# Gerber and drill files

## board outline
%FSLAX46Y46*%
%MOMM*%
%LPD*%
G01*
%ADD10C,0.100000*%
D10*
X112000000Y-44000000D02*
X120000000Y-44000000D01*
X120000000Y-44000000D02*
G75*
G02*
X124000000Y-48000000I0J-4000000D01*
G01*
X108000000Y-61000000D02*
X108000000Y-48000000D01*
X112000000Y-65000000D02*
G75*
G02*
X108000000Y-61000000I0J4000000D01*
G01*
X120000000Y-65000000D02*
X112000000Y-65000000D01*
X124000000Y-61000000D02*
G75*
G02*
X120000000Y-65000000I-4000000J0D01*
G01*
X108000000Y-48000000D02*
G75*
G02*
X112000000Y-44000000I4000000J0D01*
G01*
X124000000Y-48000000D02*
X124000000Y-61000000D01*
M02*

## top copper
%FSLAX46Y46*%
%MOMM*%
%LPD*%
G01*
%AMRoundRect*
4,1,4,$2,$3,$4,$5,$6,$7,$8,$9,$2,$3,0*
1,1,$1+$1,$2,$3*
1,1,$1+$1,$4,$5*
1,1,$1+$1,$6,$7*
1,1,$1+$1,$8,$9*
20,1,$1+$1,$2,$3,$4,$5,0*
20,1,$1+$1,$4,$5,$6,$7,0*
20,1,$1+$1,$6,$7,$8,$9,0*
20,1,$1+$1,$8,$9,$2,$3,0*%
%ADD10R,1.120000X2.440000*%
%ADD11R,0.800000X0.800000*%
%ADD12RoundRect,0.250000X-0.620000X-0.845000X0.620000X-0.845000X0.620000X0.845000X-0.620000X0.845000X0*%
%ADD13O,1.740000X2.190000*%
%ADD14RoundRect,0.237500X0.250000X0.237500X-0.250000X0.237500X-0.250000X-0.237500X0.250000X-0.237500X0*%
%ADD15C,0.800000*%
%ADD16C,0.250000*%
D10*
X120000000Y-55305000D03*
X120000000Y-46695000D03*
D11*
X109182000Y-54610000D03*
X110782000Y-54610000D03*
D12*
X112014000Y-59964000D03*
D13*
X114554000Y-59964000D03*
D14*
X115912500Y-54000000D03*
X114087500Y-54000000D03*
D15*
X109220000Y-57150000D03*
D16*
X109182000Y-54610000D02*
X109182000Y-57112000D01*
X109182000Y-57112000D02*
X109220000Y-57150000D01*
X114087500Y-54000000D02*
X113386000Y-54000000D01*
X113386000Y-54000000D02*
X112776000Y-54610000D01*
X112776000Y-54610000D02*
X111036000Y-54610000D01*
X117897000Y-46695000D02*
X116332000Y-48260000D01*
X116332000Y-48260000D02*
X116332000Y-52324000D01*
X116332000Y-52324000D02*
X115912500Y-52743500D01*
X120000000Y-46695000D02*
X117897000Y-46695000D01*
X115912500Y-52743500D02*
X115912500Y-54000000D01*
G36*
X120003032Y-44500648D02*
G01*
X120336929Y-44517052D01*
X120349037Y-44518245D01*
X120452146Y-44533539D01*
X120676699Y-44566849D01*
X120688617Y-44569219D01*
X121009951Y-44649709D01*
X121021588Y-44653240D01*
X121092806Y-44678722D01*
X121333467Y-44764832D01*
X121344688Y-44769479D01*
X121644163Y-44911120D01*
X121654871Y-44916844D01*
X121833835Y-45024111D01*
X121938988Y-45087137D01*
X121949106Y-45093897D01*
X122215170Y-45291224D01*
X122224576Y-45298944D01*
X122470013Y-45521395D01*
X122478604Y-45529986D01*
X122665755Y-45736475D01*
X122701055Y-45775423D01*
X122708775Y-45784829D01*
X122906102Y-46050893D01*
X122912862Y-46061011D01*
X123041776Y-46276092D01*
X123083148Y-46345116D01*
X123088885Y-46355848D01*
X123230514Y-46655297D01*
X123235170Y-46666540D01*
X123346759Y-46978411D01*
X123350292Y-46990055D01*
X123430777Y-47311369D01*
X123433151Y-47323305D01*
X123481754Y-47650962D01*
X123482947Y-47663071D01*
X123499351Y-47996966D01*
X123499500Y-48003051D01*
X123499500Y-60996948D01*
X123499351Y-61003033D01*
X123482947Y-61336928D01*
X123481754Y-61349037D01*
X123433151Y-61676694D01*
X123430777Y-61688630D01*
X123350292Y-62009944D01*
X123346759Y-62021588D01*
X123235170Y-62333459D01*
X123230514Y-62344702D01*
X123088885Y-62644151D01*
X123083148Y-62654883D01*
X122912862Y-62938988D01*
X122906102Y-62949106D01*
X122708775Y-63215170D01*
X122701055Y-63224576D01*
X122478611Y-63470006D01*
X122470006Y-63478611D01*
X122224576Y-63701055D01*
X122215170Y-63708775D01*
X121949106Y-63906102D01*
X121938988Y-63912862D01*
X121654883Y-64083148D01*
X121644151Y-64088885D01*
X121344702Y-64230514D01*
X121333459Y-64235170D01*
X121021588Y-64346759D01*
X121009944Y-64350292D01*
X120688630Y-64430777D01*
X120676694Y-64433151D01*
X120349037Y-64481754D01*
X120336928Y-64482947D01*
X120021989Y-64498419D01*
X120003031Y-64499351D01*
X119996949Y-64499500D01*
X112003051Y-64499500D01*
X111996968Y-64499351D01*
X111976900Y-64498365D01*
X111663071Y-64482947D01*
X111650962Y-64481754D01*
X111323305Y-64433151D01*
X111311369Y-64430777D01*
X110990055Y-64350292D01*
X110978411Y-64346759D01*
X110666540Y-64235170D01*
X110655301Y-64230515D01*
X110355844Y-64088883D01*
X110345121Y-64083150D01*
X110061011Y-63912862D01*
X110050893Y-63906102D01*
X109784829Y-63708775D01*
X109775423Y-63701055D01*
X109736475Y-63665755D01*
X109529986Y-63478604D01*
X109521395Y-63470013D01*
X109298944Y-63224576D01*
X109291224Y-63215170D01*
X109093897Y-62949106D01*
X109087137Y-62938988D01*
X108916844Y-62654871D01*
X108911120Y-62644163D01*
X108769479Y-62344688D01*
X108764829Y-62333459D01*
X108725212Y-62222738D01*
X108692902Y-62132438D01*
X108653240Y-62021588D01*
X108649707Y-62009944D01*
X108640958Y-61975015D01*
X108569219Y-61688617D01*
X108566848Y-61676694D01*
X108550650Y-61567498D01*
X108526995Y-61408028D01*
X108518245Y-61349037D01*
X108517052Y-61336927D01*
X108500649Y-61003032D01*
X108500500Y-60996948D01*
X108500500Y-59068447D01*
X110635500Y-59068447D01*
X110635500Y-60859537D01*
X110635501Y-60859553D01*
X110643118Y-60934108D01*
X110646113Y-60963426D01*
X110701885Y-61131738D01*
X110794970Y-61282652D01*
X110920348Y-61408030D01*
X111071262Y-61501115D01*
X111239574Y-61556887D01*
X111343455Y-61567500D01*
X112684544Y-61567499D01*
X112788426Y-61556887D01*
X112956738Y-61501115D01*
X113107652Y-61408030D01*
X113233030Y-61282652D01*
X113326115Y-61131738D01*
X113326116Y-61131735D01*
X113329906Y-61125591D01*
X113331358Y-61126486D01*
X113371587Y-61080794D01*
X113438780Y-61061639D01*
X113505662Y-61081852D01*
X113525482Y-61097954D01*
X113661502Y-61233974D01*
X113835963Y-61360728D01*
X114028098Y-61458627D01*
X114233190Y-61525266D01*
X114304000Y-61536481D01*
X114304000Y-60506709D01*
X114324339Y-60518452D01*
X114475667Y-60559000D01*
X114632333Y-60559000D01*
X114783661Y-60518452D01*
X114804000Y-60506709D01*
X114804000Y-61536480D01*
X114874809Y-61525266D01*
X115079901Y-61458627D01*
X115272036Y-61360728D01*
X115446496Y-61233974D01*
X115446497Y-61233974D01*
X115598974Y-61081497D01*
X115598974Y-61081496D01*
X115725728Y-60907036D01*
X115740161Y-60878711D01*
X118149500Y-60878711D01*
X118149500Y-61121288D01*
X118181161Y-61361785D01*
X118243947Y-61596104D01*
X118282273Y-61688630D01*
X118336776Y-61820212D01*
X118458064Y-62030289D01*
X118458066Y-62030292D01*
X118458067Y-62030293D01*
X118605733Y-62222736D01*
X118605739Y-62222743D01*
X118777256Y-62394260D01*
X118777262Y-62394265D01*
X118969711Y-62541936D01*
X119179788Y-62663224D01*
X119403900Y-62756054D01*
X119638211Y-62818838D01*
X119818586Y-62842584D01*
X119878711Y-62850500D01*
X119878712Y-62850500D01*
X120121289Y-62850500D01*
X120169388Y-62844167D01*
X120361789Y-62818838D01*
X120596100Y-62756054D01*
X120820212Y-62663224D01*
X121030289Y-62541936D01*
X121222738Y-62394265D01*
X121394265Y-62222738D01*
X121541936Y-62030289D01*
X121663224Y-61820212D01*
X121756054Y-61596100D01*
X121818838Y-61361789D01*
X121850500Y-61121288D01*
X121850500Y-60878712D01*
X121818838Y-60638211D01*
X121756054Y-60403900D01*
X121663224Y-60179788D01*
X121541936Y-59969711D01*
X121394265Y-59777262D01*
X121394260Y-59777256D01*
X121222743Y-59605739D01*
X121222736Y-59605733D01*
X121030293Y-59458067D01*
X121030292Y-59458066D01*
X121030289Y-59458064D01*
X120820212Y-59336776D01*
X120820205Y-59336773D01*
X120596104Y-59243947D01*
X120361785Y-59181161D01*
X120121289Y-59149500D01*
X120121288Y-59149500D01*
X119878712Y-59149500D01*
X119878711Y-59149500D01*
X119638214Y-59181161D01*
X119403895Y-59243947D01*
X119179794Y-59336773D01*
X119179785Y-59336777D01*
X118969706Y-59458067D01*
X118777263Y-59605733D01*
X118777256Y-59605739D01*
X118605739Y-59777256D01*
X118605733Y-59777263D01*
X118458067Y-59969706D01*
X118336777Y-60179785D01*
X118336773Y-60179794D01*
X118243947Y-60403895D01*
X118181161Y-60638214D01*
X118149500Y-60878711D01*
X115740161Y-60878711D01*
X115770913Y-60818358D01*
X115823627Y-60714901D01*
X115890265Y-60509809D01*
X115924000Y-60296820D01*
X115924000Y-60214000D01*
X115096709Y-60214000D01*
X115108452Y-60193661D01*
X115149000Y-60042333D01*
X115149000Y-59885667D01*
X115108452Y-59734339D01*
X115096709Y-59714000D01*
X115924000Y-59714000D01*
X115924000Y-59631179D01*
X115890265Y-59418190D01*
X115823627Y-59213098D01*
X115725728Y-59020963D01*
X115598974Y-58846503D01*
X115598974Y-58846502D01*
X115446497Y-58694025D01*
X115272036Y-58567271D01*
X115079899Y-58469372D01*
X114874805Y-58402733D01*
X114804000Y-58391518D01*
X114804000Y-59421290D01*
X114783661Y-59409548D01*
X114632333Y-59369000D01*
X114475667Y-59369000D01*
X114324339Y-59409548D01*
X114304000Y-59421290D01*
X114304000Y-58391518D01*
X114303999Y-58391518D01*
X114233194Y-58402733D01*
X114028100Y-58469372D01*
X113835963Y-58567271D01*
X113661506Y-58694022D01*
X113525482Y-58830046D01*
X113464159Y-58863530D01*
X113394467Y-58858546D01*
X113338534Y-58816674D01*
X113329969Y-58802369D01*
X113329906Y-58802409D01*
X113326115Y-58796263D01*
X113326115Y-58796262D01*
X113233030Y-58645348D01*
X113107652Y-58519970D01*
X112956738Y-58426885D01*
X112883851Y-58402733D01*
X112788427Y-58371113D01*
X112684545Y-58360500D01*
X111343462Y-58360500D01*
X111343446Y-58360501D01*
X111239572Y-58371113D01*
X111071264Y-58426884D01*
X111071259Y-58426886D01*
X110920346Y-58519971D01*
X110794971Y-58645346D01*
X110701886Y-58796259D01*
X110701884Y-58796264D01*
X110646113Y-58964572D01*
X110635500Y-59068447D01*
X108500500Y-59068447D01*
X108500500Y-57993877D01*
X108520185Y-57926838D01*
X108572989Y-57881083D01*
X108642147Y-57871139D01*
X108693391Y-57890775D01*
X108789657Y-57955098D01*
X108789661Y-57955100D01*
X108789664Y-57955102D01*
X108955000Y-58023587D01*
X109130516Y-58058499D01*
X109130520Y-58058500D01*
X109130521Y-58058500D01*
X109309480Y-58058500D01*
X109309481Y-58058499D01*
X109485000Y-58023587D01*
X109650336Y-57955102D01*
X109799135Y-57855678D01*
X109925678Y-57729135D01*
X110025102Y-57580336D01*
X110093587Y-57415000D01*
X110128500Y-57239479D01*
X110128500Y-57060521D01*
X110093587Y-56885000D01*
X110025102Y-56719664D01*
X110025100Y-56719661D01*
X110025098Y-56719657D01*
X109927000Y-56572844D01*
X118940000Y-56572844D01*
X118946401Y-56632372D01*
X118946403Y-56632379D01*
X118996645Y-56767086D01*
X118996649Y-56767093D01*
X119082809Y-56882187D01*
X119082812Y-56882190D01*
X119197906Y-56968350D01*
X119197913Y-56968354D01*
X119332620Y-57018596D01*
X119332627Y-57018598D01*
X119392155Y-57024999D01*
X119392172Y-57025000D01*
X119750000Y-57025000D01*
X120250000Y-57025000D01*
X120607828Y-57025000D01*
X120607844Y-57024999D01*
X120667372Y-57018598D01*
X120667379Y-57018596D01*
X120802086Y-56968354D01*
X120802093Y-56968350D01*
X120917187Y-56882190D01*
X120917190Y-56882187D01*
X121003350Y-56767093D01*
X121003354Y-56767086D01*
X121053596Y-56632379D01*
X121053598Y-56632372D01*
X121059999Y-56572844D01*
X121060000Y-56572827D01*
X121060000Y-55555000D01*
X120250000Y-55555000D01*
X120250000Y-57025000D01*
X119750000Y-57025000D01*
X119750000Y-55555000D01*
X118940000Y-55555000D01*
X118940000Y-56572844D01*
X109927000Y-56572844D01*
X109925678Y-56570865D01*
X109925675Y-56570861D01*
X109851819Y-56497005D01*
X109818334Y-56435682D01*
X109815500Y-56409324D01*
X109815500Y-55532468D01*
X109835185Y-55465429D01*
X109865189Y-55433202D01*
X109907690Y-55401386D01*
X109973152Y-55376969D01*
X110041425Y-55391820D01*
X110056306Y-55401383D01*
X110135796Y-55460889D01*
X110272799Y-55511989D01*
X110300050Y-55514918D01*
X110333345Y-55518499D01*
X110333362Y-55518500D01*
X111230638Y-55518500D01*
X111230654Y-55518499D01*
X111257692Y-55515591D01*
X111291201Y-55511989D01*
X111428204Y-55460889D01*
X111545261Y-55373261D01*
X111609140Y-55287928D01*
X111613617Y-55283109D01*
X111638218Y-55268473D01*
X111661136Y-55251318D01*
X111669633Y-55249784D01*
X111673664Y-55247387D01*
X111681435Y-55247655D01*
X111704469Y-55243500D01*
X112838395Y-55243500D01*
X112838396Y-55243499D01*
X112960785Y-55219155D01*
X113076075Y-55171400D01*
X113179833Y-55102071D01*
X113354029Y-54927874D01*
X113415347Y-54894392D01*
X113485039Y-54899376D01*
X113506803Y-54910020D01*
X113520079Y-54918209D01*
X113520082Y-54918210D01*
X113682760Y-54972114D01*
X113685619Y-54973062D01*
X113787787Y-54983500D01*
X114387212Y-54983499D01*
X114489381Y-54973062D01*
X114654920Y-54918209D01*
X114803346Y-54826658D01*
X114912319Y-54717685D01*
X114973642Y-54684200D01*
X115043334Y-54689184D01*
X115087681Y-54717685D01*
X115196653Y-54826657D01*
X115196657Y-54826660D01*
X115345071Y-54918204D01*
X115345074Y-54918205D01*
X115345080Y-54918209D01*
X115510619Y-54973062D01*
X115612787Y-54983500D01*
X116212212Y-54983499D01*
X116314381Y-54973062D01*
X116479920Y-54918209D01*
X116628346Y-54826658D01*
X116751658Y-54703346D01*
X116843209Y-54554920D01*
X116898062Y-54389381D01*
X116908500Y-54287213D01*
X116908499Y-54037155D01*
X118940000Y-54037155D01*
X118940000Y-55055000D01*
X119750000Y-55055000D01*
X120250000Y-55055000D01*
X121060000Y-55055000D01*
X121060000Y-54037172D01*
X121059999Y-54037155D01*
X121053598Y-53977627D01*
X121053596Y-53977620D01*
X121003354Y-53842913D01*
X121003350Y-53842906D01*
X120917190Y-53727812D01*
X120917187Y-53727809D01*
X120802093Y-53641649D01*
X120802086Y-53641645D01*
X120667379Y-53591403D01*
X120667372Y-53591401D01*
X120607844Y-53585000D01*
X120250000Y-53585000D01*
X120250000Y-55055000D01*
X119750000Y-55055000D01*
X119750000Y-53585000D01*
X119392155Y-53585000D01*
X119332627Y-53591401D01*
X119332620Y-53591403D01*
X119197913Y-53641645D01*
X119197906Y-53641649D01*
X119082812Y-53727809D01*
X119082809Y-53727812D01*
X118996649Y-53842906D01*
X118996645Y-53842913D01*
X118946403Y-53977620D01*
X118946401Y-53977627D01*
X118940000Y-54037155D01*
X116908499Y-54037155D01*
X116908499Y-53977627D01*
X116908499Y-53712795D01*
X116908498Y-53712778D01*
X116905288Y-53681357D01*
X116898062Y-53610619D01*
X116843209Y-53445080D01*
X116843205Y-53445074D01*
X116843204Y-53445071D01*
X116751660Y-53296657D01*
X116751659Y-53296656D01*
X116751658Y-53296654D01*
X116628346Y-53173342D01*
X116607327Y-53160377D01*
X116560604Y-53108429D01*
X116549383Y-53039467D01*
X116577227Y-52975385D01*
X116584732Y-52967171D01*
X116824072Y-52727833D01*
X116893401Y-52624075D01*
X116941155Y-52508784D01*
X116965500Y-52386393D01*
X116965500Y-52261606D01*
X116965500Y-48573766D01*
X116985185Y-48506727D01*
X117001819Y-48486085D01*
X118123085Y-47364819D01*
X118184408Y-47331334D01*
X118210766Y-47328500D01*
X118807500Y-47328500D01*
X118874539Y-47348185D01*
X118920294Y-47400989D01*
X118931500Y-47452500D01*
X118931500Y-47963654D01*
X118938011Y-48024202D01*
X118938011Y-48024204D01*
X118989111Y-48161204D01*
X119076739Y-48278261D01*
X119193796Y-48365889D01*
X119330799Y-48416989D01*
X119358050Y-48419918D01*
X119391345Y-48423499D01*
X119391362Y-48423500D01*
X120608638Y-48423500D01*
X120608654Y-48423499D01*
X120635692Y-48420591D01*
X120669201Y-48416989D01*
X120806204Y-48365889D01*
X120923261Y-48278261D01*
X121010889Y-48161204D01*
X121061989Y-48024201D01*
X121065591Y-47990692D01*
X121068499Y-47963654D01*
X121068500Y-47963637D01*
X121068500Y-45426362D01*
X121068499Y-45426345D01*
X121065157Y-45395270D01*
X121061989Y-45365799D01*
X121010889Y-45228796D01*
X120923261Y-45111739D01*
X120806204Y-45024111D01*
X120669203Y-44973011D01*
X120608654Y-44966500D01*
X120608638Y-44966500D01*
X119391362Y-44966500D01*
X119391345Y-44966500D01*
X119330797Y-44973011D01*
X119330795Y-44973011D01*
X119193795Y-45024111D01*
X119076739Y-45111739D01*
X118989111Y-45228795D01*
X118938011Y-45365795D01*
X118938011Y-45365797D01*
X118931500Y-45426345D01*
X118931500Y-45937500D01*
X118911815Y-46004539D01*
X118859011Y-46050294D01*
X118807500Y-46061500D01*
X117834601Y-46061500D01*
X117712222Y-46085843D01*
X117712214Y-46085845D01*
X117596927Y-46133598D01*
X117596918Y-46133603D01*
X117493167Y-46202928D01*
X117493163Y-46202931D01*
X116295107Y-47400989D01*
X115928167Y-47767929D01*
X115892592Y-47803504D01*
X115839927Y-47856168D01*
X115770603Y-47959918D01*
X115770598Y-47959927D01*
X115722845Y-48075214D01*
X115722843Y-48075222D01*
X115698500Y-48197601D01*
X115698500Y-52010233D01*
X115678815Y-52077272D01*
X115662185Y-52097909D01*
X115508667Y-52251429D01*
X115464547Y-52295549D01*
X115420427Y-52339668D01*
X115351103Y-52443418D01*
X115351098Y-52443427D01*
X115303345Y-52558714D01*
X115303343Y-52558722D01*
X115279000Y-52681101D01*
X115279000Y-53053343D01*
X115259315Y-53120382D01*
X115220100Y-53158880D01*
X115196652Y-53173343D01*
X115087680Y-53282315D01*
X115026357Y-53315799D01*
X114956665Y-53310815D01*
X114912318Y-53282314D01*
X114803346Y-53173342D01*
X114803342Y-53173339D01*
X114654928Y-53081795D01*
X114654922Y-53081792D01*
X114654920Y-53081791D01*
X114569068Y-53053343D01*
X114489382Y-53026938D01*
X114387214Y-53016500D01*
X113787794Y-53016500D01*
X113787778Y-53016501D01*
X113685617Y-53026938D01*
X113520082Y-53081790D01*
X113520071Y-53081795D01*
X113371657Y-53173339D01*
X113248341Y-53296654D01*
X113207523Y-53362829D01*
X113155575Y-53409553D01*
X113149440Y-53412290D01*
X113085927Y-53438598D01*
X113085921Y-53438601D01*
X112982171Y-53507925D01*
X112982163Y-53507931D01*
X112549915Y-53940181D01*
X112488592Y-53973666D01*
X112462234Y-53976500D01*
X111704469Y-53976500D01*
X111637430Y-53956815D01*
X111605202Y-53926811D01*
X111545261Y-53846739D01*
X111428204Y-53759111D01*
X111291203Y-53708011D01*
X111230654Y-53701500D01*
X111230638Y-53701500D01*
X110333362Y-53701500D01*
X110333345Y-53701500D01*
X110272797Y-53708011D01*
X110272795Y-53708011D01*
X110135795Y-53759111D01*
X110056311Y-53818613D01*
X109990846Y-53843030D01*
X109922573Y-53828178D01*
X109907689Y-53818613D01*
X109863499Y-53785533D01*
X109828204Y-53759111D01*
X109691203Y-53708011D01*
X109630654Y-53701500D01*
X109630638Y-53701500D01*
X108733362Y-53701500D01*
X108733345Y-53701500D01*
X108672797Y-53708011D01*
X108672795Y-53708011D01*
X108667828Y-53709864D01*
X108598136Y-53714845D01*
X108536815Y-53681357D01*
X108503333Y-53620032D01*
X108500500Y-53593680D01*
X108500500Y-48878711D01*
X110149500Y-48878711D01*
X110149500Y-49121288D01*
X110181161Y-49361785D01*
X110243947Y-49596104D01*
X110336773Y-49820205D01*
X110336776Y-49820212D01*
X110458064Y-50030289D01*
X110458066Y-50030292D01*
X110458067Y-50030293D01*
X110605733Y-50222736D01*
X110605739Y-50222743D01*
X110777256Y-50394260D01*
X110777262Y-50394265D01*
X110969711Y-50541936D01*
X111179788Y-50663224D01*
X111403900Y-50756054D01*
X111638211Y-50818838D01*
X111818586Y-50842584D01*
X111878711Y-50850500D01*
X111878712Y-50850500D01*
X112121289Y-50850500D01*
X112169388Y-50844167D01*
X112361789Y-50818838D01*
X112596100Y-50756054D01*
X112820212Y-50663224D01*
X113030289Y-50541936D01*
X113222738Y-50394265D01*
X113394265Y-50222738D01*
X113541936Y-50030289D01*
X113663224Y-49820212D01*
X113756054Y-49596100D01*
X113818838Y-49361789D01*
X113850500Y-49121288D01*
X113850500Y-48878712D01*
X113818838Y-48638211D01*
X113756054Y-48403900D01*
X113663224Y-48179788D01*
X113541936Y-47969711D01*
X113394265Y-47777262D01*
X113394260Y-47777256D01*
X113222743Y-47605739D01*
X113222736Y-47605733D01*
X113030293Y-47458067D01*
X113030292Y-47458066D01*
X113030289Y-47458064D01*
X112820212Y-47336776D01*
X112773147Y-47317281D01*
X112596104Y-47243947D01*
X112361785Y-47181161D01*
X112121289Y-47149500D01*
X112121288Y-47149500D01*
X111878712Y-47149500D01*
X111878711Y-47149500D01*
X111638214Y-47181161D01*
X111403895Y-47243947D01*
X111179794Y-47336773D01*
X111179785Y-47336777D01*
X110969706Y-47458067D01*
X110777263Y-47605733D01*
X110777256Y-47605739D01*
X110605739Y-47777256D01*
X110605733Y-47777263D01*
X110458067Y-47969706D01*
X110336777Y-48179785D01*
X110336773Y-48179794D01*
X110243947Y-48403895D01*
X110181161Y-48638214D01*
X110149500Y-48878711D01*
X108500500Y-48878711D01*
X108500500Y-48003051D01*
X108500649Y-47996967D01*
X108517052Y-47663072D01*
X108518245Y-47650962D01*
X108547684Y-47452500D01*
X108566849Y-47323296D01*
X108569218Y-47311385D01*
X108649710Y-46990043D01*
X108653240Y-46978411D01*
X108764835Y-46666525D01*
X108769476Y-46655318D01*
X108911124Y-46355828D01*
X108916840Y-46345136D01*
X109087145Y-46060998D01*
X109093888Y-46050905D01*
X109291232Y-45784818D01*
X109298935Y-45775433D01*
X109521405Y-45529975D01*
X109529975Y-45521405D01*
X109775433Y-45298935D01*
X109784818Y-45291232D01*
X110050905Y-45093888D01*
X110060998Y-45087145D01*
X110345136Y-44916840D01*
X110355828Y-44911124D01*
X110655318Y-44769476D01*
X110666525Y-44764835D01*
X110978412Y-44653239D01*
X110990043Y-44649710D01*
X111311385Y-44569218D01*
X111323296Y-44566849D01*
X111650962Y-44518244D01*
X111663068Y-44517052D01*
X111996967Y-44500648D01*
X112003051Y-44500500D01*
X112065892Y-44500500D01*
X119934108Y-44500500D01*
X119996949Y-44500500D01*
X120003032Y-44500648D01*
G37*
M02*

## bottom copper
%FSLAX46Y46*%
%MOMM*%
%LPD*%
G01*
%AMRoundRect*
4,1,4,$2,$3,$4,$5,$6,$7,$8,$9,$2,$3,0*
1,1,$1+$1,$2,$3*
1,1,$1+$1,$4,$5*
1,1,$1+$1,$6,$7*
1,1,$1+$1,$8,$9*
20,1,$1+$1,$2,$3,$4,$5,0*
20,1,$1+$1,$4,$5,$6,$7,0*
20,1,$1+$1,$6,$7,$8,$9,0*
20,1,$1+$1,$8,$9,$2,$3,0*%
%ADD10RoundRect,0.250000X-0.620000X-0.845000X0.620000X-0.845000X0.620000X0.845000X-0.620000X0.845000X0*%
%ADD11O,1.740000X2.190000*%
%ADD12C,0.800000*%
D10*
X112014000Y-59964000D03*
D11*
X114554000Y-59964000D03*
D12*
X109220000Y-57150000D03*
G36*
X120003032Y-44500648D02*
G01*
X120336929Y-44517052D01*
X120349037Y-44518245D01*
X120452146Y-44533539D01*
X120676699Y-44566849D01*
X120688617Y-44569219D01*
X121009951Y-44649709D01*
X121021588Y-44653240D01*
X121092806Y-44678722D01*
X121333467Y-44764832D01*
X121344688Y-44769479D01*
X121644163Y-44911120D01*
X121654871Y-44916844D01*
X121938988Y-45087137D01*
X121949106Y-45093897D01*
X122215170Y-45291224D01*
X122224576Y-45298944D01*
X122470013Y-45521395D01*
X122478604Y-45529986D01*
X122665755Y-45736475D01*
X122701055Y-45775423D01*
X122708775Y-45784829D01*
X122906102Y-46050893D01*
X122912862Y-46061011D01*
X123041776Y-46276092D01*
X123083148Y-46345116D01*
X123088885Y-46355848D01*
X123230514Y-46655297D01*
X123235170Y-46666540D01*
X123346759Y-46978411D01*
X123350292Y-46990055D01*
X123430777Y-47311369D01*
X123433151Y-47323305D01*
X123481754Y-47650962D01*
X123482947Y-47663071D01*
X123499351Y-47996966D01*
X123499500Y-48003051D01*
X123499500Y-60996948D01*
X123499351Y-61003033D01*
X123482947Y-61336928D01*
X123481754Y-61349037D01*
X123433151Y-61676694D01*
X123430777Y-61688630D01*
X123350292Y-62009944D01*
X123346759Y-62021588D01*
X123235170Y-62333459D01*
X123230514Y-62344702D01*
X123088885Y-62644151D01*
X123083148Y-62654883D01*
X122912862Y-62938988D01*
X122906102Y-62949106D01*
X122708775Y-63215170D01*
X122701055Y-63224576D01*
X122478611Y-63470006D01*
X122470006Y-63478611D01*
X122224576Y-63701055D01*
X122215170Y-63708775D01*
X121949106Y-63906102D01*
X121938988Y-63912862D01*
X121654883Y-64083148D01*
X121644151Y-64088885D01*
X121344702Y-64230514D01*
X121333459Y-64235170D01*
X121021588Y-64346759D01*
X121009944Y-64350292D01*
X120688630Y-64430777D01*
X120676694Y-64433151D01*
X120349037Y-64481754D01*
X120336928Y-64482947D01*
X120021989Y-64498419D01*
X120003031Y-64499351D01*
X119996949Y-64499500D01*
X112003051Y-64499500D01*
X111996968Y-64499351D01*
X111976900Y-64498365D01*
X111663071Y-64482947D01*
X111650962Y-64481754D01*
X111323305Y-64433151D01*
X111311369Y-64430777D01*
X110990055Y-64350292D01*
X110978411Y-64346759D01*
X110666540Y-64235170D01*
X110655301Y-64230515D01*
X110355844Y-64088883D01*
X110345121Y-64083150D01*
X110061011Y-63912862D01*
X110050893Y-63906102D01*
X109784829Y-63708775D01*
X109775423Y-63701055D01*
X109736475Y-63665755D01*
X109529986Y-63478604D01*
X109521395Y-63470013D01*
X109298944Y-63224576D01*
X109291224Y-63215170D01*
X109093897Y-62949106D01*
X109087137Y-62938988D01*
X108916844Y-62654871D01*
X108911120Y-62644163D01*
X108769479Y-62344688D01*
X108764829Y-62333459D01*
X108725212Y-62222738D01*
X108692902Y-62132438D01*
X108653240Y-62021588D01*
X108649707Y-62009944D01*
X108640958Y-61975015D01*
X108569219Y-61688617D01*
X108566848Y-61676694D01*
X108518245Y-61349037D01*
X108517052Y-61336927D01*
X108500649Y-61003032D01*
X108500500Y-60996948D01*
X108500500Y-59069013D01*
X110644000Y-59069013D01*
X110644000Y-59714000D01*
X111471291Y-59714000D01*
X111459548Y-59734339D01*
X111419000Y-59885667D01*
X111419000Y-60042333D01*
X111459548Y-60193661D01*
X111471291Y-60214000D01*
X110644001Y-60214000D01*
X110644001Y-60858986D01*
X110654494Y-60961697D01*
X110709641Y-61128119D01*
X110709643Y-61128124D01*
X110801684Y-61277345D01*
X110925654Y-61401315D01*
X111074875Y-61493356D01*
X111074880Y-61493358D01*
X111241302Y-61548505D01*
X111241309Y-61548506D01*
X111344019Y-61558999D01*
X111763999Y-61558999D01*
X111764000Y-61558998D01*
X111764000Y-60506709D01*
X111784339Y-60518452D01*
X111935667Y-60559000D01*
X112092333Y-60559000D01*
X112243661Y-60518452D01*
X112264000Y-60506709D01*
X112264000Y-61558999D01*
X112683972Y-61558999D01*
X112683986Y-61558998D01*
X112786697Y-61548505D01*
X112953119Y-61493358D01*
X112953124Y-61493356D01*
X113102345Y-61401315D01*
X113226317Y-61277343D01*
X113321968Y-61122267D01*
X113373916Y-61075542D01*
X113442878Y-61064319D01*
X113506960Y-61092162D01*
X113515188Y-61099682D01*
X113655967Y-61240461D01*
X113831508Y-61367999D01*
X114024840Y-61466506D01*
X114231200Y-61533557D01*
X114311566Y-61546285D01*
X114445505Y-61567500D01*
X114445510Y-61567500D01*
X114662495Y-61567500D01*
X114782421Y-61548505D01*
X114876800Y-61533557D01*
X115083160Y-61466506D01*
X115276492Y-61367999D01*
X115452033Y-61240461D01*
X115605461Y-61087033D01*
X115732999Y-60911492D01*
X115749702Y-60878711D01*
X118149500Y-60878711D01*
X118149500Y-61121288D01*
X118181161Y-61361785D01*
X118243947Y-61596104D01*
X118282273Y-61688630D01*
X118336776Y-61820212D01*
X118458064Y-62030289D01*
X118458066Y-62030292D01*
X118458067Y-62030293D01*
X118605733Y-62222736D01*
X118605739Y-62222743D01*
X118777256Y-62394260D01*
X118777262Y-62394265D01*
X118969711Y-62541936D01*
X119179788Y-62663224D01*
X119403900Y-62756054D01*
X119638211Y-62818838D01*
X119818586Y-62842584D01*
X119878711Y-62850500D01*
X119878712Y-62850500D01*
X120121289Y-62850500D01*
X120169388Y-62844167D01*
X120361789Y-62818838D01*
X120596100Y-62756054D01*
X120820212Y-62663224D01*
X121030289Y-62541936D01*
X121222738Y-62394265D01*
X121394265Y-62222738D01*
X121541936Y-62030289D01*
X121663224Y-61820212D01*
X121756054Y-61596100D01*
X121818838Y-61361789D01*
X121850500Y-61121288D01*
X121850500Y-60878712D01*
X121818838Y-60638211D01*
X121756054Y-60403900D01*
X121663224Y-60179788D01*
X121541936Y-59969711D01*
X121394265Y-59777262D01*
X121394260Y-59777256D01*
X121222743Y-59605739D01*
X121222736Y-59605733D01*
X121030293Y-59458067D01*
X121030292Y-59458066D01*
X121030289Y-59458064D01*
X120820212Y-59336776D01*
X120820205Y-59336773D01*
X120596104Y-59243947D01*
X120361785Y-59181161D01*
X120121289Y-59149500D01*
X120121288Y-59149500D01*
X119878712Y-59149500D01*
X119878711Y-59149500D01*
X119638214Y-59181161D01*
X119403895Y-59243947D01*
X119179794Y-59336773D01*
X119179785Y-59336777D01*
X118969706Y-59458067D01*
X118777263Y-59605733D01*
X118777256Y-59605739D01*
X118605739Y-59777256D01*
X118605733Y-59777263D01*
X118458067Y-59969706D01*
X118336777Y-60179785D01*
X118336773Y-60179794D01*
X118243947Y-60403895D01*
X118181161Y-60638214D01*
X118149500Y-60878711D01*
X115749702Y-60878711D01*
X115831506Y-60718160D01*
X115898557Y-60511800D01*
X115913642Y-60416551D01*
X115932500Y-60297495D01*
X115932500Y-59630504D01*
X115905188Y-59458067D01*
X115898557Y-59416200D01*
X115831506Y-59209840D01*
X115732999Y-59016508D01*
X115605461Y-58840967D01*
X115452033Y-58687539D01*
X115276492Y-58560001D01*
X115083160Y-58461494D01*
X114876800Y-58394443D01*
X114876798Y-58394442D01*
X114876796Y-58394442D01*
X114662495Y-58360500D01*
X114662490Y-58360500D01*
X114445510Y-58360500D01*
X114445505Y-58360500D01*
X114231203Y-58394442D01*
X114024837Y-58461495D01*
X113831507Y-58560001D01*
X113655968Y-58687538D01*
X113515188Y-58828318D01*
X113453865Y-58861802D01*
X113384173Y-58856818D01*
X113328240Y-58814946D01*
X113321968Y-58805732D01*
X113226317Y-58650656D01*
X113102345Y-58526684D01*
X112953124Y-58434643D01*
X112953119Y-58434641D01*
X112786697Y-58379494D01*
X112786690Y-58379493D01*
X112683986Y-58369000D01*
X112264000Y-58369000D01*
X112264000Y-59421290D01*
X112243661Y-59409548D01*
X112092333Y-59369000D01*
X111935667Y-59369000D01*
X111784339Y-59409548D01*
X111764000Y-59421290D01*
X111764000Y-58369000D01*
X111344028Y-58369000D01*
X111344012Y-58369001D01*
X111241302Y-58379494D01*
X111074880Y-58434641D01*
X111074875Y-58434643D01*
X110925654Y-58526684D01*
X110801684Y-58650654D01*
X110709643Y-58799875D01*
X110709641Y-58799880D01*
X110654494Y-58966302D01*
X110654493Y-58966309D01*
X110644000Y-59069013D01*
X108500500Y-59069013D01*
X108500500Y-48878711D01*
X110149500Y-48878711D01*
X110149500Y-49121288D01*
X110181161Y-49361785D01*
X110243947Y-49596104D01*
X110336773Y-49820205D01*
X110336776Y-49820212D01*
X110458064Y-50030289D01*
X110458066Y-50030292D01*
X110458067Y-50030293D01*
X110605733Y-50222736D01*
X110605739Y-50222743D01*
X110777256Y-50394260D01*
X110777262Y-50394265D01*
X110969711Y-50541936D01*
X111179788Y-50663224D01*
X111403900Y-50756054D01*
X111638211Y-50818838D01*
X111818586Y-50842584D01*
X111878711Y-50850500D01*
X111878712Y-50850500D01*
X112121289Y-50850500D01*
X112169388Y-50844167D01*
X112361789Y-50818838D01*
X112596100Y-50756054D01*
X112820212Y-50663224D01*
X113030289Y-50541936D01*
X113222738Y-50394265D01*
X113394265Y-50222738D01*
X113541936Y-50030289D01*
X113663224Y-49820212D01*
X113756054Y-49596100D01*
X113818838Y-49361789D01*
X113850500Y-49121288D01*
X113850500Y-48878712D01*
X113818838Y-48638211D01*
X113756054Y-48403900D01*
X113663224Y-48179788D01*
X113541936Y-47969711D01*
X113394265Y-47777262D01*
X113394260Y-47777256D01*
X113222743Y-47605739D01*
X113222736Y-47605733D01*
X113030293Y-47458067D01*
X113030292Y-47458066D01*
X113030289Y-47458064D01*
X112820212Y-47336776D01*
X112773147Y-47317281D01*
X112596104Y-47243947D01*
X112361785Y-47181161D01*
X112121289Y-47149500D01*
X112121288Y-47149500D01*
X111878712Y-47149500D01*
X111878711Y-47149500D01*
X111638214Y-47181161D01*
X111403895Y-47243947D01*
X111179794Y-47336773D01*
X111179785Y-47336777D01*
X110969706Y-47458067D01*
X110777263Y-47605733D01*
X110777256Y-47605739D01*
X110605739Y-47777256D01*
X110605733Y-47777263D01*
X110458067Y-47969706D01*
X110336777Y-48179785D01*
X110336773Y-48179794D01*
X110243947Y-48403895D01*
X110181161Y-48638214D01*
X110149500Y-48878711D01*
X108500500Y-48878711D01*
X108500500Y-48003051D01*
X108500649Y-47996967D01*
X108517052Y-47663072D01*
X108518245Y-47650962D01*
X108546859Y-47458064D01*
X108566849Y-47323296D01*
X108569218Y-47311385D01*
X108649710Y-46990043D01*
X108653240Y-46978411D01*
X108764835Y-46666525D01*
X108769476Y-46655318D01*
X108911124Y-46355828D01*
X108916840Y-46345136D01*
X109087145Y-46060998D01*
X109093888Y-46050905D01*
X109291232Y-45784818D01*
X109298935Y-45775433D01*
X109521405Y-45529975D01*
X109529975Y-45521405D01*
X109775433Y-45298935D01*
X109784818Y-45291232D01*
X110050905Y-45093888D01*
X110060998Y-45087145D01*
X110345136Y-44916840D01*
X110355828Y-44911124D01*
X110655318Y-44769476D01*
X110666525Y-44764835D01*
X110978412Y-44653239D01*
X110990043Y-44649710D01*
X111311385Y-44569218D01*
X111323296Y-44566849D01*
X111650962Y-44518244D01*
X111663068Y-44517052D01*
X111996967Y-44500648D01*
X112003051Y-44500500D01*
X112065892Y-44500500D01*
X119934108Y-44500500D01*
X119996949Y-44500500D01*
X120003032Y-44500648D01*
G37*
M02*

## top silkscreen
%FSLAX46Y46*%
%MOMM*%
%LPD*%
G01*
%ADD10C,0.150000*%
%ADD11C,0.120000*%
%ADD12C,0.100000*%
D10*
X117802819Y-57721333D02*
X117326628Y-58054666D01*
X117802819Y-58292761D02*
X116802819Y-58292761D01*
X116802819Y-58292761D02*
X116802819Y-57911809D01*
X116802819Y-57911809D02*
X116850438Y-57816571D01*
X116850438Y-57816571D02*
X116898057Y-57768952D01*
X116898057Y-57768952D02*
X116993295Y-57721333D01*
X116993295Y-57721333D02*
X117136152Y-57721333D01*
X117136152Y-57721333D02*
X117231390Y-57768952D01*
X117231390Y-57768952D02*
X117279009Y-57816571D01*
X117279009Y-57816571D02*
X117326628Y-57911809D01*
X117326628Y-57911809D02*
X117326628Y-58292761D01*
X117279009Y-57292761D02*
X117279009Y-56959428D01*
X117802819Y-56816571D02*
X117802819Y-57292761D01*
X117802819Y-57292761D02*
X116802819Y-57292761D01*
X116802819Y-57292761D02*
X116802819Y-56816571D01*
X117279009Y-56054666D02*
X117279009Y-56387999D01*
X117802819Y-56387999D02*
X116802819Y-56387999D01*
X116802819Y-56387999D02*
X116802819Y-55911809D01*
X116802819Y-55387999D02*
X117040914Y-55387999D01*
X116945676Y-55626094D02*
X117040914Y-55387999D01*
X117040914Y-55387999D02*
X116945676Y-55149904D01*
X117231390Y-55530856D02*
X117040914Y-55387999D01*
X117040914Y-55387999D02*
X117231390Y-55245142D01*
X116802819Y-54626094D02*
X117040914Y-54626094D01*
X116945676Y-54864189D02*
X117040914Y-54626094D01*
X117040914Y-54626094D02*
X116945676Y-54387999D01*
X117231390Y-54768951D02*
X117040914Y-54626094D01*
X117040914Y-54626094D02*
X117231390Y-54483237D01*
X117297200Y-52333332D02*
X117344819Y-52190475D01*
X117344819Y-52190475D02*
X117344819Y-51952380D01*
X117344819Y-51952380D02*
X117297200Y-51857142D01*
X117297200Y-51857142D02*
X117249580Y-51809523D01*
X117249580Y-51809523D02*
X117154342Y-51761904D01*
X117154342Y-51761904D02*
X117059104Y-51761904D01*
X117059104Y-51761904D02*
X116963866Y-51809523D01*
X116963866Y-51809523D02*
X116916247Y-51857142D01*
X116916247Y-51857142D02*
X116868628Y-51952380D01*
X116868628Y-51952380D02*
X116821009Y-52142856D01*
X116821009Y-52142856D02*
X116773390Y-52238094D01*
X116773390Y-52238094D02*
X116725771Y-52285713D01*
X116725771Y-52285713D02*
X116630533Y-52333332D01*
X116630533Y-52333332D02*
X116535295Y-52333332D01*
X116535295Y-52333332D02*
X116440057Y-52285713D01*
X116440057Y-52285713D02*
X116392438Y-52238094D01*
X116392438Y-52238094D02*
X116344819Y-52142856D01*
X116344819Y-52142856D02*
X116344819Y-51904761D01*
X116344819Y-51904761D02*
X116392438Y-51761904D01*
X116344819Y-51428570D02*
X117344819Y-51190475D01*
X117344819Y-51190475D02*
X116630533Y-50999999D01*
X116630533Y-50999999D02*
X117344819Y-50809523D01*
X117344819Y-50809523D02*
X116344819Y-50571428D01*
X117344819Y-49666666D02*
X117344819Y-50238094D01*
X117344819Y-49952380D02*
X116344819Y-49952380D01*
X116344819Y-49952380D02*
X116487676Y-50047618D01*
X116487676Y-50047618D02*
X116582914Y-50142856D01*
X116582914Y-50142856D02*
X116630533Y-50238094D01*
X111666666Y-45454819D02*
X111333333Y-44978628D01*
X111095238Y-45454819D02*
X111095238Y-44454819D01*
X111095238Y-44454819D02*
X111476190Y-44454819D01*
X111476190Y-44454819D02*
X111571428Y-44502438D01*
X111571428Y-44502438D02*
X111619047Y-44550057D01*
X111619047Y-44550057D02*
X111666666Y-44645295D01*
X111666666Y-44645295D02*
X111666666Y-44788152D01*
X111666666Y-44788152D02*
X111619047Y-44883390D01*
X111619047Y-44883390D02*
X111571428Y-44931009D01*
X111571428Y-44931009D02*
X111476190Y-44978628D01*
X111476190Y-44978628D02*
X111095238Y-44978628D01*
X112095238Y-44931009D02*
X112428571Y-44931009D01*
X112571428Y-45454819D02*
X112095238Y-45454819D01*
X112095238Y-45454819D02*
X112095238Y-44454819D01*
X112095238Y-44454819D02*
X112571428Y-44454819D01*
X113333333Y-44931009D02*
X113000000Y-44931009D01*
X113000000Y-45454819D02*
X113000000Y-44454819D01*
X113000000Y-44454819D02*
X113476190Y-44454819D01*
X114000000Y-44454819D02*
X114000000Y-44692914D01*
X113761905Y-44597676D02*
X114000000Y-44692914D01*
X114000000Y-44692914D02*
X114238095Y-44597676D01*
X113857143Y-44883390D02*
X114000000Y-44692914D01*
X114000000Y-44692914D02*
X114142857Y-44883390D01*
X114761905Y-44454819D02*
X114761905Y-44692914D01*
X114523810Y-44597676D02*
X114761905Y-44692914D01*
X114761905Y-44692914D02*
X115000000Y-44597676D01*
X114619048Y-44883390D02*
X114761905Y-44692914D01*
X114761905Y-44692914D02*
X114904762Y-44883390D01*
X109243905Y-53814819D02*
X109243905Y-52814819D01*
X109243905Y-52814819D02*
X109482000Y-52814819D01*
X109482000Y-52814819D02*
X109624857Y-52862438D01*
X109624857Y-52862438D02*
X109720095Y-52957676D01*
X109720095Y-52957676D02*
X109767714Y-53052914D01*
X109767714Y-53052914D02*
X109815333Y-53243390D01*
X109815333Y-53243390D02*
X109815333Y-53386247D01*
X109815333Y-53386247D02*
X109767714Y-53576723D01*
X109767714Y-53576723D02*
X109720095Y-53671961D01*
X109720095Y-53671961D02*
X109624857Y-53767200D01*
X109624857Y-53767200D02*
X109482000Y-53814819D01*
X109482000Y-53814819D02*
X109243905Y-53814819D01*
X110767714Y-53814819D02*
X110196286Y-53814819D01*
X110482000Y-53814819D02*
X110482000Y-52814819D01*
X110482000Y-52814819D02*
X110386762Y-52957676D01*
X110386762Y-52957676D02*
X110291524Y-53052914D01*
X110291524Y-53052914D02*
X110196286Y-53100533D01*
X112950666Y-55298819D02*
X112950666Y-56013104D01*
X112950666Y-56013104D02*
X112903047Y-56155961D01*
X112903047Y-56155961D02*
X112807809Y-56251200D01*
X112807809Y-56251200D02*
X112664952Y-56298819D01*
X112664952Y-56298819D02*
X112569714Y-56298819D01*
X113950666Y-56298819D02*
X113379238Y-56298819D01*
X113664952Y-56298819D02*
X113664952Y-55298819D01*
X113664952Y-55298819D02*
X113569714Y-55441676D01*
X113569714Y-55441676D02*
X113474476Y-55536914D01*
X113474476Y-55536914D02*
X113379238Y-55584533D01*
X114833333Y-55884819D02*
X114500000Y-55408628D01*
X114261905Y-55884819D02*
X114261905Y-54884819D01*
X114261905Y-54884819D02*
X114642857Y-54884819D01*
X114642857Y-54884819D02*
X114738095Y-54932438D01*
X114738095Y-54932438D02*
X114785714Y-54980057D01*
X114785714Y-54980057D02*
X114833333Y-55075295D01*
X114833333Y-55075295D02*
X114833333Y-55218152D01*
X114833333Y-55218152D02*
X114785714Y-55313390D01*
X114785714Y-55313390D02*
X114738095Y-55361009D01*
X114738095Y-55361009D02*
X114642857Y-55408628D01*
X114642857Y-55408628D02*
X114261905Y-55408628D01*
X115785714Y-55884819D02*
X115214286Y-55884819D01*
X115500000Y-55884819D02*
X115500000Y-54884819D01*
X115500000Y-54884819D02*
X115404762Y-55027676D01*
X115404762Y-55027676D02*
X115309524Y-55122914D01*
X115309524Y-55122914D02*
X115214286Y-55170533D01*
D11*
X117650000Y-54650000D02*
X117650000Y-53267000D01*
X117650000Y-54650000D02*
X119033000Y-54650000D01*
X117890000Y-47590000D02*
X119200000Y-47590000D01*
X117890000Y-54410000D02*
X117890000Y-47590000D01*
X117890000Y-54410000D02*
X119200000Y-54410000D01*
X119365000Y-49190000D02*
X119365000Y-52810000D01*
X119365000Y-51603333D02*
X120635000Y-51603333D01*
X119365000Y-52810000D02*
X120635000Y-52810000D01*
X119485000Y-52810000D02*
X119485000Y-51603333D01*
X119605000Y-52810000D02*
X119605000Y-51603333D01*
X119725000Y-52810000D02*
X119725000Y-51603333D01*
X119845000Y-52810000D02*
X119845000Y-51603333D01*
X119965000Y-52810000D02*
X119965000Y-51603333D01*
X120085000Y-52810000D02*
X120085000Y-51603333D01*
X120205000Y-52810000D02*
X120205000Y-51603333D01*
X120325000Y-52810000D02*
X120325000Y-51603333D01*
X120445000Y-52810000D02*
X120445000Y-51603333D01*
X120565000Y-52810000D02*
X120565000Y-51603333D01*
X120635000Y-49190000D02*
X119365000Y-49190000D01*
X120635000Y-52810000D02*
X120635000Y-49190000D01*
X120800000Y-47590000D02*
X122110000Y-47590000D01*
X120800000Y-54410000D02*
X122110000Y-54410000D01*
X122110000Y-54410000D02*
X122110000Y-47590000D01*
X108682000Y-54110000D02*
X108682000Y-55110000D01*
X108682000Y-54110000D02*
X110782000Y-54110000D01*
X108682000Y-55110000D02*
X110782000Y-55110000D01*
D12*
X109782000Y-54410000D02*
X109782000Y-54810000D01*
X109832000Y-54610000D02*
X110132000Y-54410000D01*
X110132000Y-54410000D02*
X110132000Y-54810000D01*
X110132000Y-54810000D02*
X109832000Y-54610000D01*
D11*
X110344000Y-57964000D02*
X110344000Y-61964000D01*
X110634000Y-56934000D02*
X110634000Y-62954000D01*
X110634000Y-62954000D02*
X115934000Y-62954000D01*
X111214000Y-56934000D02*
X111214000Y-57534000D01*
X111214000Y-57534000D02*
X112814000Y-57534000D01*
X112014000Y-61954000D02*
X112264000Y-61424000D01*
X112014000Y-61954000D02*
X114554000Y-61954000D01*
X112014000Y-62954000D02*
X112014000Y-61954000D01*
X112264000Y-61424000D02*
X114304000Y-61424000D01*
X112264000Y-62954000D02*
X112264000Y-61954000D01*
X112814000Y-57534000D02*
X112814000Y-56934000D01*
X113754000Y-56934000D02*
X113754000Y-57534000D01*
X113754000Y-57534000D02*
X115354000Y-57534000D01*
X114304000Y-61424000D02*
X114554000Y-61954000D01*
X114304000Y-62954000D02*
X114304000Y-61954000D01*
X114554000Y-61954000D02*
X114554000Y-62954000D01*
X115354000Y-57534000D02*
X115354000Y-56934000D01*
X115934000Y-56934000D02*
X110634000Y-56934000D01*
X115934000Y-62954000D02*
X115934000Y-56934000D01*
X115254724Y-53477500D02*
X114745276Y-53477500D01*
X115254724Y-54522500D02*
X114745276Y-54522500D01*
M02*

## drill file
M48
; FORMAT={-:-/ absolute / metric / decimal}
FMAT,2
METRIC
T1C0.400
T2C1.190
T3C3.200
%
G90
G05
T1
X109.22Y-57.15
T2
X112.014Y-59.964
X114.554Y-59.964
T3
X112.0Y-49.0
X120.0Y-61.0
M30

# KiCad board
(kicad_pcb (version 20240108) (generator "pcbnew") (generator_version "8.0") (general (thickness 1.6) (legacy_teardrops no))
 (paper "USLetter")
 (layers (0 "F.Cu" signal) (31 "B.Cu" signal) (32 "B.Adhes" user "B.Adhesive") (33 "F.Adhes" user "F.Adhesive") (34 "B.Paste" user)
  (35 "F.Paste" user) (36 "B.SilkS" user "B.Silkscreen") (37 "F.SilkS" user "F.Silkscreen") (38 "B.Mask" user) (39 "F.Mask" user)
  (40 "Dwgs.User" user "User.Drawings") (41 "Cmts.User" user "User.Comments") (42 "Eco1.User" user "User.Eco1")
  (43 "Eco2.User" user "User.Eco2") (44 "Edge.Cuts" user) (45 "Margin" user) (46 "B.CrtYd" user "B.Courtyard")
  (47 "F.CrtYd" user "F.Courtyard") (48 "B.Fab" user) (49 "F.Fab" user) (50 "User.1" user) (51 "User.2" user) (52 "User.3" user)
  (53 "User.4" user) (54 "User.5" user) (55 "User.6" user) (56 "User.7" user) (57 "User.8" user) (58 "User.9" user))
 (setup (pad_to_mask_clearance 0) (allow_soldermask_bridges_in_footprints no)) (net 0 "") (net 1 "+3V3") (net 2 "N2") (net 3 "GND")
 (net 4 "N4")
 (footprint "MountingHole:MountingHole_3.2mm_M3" (layer "F.Cu") (at 120 61)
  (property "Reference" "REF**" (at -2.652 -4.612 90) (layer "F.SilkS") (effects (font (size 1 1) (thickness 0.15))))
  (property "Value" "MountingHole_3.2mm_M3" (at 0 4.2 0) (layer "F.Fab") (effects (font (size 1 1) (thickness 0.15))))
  (pad "" np_thru_hole circle (at 0 0) (size 3.2 3.2) (drill 3.2) (layers "*.Cu" "*.Mask")))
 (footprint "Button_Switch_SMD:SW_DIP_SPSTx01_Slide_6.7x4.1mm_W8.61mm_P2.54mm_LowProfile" (layer "F.Cu") (at 120 51 90)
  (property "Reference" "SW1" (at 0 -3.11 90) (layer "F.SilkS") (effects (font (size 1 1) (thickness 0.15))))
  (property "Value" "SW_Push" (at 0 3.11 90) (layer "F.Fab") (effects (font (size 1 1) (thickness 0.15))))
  (fp_line (start -3.65 -2.35) (end -2.267 -2.35) (stroke (width 0.12) (type solid)) (layer "F.SilkS"))
  (fp_line (start -3.65 -2.35) (end -3.65 -0.967) (stroke (width 0.12) (type solid)) (layer "F.SilkS"))
  (fp_line (start 3.41 -2.11) (end 3.41 -0.8) (stroke (width 0.12) (type solid)) (layer "F.SilkS"))
  (fp_line (start -3.41 -2.11) (end 3.41 -2.11) (stroke (width 0.12) (type solid)) (layer "F.SilkS"))
  (fp_line (start -3.41 -2.11) (end -3.41 -0.8) (stroke (width 0.12) (type solid)) (layer "F.SilkS"))
  (fp_line (start 1.81 -0.635) (end -1.81 -0.635) (stroke (width 0.12) (type solid)) (layer "F.SilkS"))
  (fp_line (start -0.603333 -0.635) (end -0.603333 0.635) (stroke (width 0.12) (type solid)) (layer "F.SilkS"))
  (fp_line (start -1.81 -0.635) (end -1.81 0.635) (stroke (width 0.12) (type solid)) (layer "F.SilkS"))
  (fp_line (start -1.81 -0.515) (end -0.603333 -0.515) (stroke (width 0.12) (type solid)) (layer "F.SilkS"))
  (fp_line (start -1.81 -0.395) (end -0.603333 -0.395) (stroke (width 0.12) (type solid)) (layer "F.SilkS"))
  (fp_line (start -1.81 -0.275) (end -0.603333 -0.275) (stroke (width 0.12) (type solid)) (layer "F.SilkS"))
  (fp_line (start -1.81 -0.155) (end -0.603333 -0.155) (stroke (width 0.12) (type solid)) (layer "F.SilkS"))
  (fp_line (start -1.81 -0.035) (end -0.603333 -0.035) (stroke (width 0.12) (type solid)) (layer "F.SilkS"))
  (fp_line (start -1.81 0.085) (end -0.603333 0.085) (stroke (width 0.12) (type solid)) (layer "F.SilkS"))
  (fp_line (start -1.81 0.205) (end -0.603333 0.205) (stroke (width 0.12) (type solid)) (layer "F.SilkS"))
  (fp_line (start -1.81 0.325) (end -0.603333 0.325) (stroke (width 0.12) (type solid)) (layer "F.SilkS"))
  (fp_line (start -1.81 0.445) (end -0.603333 0.445) (stroke (width 0.12) (type solid)) (layer "F.SilkS"))
  (fp_line (start -1.81 0.565) (end -0.603333 0.565) (stroke (width 0.12) (type solid)) (layer "F.SilkS"))
  (fp_line (start 1.81 0.635) (end 1.81 -0.635) (stroke (width 0.12) (type solid)) (layer "F.SilkS"))
  (fp_line (start -1.81 0.635) (end 1.81 0.635) (stroke (width 0.12) (type solid)) (layer "F.SilkS"))
  (fp_line (start 3.41 0.8) (end 3.41 2.11) (stroke (width 0.12) (type solid)) (layer "F.SilkS"))
  (fp_line (start -3.41 0.8) (end -3.41 2.11) (stroke (width 0.12) (type solid)) (layer "F.SilkS"))
  (fp_line (start -3.41 2.11) (end 3.41 2.11) (stroke (width 0.12) (type solid)) (layer "F.SilkS"))
  (pad "1" smd rect (at -4.305 0 90) (size 2.44 1.12) (layers "F.Cu" "F.Paste" "F.Mask") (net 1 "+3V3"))
  (pad "2" smd rect (at 4.305 0 90) (size 2.44 1.12) (layers "F.Cu" "F.Paste" "F.Mask") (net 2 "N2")))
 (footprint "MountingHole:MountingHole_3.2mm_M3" (layer "F.Cu") (at 112 49)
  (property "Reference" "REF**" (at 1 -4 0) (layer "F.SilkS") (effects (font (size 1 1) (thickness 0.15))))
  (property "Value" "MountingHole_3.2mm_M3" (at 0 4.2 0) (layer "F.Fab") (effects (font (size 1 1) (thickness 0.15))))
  (pad "" np_thru_hole circle (at 0 0) (size 3.2 3.2) (drill 3.2) (layers "*.Cu" "*.Mask")))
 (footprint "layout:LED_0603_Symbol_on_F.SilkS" (layer "F.Cu") (at 109.982 54.61)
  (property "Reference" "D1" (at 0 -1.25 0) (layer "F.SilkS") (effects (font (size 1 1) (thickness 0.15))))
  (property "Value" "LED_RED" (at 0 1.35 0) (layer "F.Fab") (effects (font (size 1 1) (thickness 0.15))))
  (fp_line (start -1.3 -0.5) (end -1.3 0.5) (stroke (width 0.12) (type solid)) (layer "F.SilkS"))
  (fp_line (start -1.3 -0.5) (end 0.8 -0.5) (stroke (width 0.12) (type solid)) (layer "F.SilkS"))
  (fp_line (start -1.3 0.5) (end 0.8 0.5) (stroke (width 0.12) (type solid)) (layer "F.SilkS"))
  (fp_line (start -0.2 -0.2) (end -0.2 0.2) (stroke (width 0.1) (type solid)) (layer "F.SilkS"))
  (fp_line (start -0.15 0) (end 0.15 -0.2) (stroke (width 0.1) (type solid)) (layer "F.SilkS"))
  (fp_line (start 0.15 -0.2) (end 0.15 0.2) (stroke (width 0.1) (type solid)) (layer "F.SilkS"))
  (fp_line (start 0.15 0.2) (end -0.15 0) (stroke (width 0.1) (type solid)) (layer "F.SilkS"))
  (pad "1" smd rect (at -0.8 0 180) (size 0.8 0.8) (layers "F.Cu" "F.Paste" "F.Mask") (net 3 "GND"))
  (pad "2" smd rect (at 0.8 0 180) (size 0.8 0.8) (layers "F.Cu" "F.Paste" "F.Mask") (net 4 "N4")))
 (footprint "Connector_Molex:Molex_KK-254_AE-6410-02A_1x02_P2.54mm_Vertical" (layer "F.Cu") (at 112.014 59.964)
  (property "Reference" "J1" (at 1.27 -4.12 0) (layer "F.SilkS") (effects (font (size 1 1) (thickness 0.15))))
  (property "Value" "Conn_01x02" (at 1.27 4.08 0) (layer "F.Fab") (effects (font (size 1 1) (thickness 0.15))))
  (fp_line (start -1.67 -2) (end -1.67 2) (stroke (width 0.12) (type solid)) (layer "F.SilkS"))
  (fp_line (start -1.38 -3.03) (end -1.38 2.99) (stroke (width 0.12) (type solid)) (layer "F.SilkS"))
  (fp_line (start -1.38 2.99) (end 3.92 2.99) (stroke (width 0.12) (type solid)) (layer "F.SilkS"))
  (fp_line (start -0.8 -3.03) (end -0.8 -2.43) (stroke (width 0.12) (type solid)) (layer "F.SilkS"))
  (fp_line (start -0.8 -2.43) (end 0.8 -2.43) (stroke (width 0.12) (type solid)) (layer "F.SilkS"))
  (fp_line (start 0 1.99) (end 0.25 1.46) (stroke (width 0.12) (type solid)) (layer "F.SilkS"))
  (fp_line (start 0 1.99) (end 2.54 1.99) (stroke (width 0.12) (type solid)) (layer "F.SilkS"))
  (fp_line (start 0 2.99) (end 0 1.99) (stroke (width 0.12) (type solid)) (layer "F.SilkS"))
  (fp_line (start 0.25 1.46) (end 2.29 1.46) (stroke (width 0.12) (type solid)) (layer "F.SilkS"))
  (fp_line (start 0.25 2.99) (end 0.25 1.99) (stroke (width 0.12) (type solid)) (layer "F.SilkS"))
  (fp_line (start 0.8 -2.43) (end 0.8 -3.03) (stroke (width 0.12) (type solid)) (layer "F.SilkS"))
  (fp_line (start 1.74 -3.03) (end 1.74 -2.43) (stroke (width 0.12) (type solid)) (layer "F.SilkS"))
  (fp_line (start 1.74 -2.43) (end 3.34 -2.43) (stroke (width 0.12) (type solid)) (layer "F.SilkS"))
  (fp_line (start 2.29 1.46) (end 2.54 1.99) (stroke (width 0.12) (type solid)) (layer "F.SilkS"))
  (fp_line (start 2.29 2.99) (end 2.29 1.99) (stroke (width 0.12) (type solid)) (layer "F.SilkS"))
  (fp_line (start 2.54 1.99) (end 2.54 2.99) (stroke (width 0.12) (type solid)) (layer "F.SilkS"))
  (fp_line (start 3.34 -2.43) (end 3.34 -3.03) (stroke (width 0.12) (type solid)) (layer "F.SilkS"))
  (fp_line (start 3.92 -3.03) (end -1.38 -3.03) (stroke (width 0.12) (type solid)) (layer "F.SilkS"))
  (fp_line (start 3.92 2.99) (end 3.92 -3.03) (stroke (width 0.12) (type solid)) (layer "F.SilkS"))
  (pad "1" thru_hole roundrect (at 0 0) (size 1.74 2.19) (drill 1.19) (layers "*.Cu" "*.Mask") (remove_unused_layers no)
   (roundrect_rratio 0.143678) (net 3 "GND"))
  (pad "2" thru_hole oval (at 2.54 0) (size 1.74 2.19) (drill 1.19) (layers "*.Cu" "*.Mask") (remove_unused_layers no) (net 1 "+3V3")))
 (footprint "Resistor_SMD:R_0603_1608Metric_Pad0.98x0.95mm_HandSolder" (layer "F.Cu") (at 115 54 180)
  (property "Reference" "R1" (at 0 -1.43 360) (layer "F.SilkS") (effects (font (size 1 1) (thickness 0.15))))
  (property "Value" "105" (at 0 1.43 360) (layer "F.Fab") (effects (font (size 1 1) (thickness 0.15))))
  (fp_line (start -0.254724 0.5225) (end 0.254724 0.5225) (stroke (width 0.12) (type solid)) (layer "F.SilkS"))
  (fp_line (start -0.254724 -0.5225) (end 0.254724 -0.5225) (stroke (width 0.12) (type solid)) (layer "F.SilkS"))
  (pad "1" smd roundrect (at -0.9125 0 180) (size 0.975 0.95) (layers "F.Cu" "F.Paste" "F.Mask") (roundrect_rratio 0.25) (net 2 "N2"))
  (pad "2" smd roundrect (at 0.9125 0 180) (size 0.975 0.95) (layers "F.Cu" "F.Paste" "F.Mask") (roundrect_rratio 0.25) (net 4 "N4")))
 (gr_line (start 112 44) (end 120 44) (stroke (width 0.1) (type default)) (layer "Edge.Cuts"))
 (gr_arc (start 120 44) (mid 122.828427 45.171573) (end 124 48) (stroke (width 0.1) (type default)) (layer "Edge.Cuts"))
 (gr_line (start 108 61) (end 108 48) (stroke (width 0.1) (type default)) (layer "Edge.Cuts"))
 (gr_arc (start 112 65) (mid 109.171573 63.828427) (end 108 61) (stroke (width 0.1) (type default)) (layer "Edge.Cuts"))
 (gr_line (start 120 65) (end 112 65) (stroke (width 0.1) (type default)) (layer "Edge.Cuts"))
 (gr_arc (start 124 61) (mid 122.828427 63.828427) (end 120 65) (stroke (width 0.1) (type default)) (layer "Edge.Cuts"))
 (gr_arc (start 108 48) (mid 109.171573 45.171573) (end 112 44) (stroke (width 0.1) (type default)) (layer "Edge.Cuts"))
 (gr_line (start 124 48) (end 124 61) (stroke (width 0.1) (type default)) (layer "Edge.Cuts"))
 (segment (start 109.182 54.61) (end 109.182 57.112) (width 0.25) (layer "F.Cu") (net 3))
 (segment (start 109.182 57.112) (end 109.22 57.15) (width 0.25) (layer "F.Cu") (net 3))
 (via (at 109.22 57.15) (size 0.8) (drill 0.4) (layers "F.Cu" "B.Cu") (free yes) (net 3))
 (segment (start 114.0875 54) (end 113.386 54) (width 0.25) (layer "F.Cu") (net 4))
 (segment (start 113.386 54) (end 112.776 54.61) (width 0.25) (layer "F.Cu") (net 4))
 (segment (start 112.776 54.61) (end 111.036 54.61) (width 0.25) (layer "F.Cu") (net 4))
 (segment (start 117.897 46.695) (end 116.332 48.26) (width 0.25) (layer "F.Cu") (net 2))
 (segment (start 116.332 48.26) (end 116.332 52.324) (width 0.25) (layer "F.Cu") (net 2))
 (segment (start 116.332 52.324) (end 115.9125 52.7435) (width 0.25) (layer "F.Cu") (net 2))
 (segment (start 120 46.695) (end 117.897 46.695) (width 0.25) (layer "F.Cu") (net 2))
 (segment (start 115.9125 52.7435) (end 115.9125 54) (width 0.25) (layer "F.Cu") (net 2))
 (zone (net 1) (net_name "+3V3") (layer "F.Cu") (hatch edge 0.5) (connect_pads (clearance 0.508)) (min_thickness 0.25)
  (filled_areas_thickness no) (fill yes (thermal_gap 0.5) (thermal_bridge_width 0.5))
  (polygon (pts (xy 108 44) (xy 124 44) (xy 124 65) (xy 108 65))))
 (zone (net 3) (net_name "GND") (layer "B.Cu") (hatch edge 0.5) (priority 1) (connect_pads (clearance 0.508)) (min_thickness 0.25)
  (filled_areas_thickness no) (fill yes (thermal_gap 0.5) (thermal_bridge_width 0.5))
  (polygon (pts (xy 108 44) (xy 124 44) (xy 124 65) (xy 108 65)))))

